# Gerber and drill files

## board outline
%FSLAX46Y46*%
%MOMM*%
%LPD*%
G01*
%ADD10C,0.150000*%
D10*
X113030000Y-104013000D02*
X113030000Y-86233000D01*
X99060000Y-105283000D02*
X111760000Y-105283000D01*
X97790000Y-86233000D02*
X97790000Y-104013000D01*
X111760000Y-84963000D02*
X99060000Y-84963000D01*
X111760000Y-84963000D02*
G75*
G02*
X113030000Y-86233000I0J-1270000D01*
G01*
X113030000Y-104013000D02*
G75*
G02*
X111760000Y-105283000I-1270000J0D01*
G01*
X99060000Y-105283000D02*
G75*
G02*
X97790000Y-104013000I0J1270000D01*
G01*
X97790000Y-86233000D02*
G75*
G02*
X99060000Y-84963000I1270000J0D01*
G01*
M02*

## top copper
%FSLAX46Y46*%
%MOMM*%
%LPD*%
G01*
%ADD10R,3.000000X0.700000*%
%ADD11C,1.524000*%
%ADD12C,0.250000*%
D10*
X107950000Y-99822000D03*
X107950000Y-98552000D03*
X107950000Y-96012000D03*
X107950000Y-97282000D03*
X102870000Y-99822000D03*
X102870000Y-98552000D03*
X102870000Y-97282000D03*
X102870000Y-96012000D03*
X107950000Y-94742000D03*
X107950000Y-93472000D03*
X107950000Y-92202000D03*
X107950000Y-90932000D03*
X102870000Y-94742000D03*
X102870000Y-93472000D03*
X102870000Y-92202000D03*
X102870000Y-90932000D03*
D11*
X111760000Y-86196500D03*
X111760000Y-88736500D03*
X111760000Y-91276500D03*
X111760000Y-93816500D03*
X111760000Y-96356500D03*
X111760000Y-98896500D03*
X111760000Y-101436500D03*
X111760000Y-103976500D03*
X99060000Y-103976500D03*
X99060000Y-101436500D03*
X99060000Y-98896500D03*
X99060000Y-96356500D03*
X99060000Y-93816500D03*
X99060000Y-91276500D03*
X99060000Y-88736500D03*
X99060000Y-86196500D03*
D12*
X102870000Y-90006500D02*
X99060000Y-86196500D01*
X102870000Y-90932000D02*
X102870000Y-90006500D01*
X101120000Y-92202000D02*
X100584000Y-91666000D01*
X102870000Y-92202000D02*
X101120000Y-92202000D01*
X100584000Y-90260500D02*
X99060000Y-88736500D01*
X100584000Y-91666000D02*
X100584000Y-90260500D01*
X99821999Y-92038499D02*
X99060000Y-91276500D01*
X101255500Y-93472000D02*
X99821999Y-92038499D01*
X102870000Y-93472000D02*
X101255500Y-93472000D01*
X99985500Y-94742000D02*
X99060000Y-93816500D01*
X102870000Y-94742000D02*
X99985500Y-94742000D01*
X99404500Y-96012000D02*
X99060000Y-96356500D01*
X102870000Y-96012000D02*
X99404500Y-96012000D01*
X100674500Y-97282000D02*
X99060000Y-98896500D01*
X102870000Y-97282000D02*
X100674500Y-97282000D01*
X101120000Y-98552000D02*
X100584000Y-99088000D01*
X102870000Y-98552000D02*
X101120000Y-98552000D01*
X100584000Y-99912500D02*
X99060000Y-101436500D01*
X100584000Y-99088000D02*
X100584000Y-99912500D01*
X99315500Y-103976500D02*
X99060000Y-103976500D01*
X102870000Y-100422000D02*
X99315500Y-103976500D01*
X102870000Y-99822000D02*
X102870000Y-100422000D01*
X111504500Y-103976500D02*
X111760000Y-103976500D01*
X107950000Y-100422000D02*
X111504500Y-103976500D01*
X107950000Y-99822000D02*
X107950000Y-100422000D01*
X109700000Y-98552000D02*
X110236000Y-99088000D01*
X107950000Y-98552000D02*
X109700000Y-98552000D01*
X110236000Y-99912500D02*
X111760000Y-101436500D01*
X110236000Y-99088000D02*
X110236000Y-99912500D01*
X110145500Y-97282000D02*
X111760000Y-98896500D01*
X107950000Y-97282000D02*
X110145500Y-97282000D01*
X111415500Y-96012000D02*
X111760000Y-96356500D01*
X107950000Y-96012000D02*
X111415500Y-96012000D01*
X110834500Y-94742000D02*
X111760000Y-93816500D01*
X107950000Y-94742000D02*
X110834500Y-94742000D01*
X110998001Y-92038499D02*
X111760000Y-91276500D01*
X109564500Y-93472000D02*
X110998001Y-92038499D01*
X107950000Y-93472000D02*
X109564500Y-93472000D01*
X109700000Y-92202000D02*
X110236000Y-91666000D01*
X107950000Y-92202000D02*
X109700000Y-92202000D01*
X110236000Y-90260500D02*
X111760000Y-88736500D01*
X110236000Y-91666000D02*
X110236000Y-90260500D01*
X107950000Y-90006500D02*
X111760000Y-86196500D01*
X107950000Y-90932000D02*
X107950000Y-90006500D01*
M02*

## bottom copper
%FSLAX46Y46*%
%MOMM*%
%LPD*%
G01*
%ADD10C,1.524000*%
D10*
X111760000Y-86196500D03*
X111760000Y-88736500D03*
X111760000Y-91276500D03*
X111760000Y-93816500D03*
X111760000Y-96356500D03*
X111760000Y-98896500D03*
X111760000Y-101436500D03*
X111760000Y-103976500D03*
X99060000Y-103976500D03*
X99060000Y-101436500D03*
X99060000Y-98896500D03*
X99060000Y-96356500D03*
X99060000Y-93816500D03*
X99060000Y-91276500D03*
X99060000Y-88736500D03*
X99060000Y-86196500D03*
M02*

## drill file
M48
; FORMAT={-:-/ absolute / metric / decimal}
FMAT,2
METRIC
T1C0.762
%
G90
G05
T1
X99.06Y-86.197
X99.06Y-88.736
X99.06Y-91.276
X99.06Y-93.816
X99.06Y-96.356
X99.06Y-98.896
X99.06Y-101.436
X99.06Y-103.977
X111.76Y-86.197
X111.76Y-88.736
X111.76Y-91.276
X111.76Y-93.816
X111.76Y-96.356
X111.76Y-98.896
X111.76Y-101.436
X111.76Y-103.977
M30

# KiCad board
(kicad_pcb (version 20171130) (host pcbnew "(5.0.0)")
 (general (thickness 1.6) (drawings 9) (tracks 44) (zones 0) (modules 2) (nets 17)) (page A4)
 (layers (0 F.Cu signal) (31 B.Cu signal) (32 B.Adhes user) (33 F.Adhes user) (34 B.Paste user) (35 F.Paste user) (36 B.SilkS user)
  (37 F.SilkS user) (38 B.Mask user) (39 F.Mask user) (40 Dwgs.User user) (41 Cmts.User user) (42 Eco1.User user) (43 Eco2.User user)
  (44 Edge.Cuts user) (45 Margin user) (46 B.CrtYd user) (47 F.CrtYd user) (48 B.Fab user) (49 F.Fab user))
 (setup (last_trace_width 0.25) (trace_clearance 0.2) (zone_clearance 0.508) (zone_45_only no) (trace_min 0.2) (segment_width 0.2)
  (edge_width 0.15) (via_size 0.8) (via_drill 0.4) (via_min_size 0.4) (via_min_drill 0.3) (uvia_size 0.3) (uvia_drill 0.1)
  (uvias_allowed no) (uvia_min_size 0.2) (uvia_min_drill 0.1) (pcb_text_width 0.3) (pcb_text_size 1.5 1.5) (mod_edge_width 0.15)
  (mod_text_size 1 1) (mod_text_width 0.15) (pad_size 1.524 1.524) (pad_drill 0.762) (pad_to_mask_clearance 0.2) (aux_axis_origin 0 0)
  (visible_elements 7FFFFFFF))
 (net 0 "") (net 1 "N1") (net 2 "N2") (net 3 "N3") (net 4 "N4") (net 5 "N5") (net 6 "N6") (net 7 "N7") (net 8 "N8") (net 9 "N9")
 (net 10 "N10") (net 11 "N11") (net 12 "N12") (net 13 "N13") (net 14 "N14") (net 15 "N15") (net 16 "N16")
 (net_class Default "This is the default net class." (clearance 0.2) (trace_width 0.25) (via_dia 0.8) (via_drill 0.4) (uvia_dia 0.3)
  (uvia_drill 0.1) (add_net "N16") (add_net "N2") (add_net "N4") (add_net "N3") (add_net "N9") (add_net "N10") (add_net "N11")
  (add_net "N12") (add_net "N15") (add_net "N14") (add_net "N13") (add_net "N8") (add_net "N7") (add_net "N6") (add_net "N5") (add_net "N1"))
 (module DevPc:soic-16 (layer F.Cu) (at 105.41 89.662)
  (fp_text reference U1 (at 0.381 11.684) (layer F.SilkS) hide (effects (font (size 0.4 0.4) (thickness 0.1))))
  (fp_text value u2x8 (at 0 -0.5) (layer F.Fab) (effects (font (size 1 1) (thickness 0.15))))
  (pad 9 smd rect (at 2.54 10.16 90) (size 0.7 3) (layers F.Cu F.Paste F.Mask) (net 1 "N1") (solder_mask_margin 0.1))
  (pad 10 smd rect (at 2.54 8.89 90) (size 0.7 3) (layers F.Cu F.Paste F.Mask) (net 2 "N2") (solder_mask_margin 0.1))
  (pad 12 smd rect (at 2.54 6.35 90) (size 0.7 3) (layers F.Cu F.Paste F.Mask) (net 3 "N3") (solder_mask_margin 0.1))
  (pad 11 smd rect (at 2.54 7.62 90) (size 0.7 3) (layers F.Cu F.Paste F.Mask) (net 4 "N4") (solder_mask_margin 0.1))
  (pad 8 smd rect (at -2.54 10.16 90) (size 0.7 3) (layers F.Cu F.Paste F.Mask) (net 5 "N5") (solder_mask_margin 0.1))
  (pad 7 smd rect (at -2.54 8.89 90) (size 0.7 3) (layers F.Cu F.Paste F.Mask) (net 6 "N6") (solder_mask_margin 0.1))
  (pad 6 smd rect (at -2.54 7.62 90) (size 0.7 3) (layers F.Cu F.Paste F.Mask) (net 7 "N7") (solder_mask_margin 0.1))
  (pad 5 smd rect (at -2.54 6.35 90) (size 0.7 3) (layers F.Cu F.Paste F.Mask) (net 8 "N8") (solder_mask_margin 0.1))
  (pad 13 smd rect (at 2.54 5.08 90) (size 0.7 3) (layers F.Cu F.Paste F.Mask) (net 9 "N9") (solder_mask_margin 0.1))
  (pad 14 smd rect (at 2.54 3.81 90) (size 0.7 3) (layers F.Cu F.Paste F.Mask) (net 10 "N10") (solder_mask_margin 0.1))
  (pad 15 smd rect (at 2.54 2.54 90) (size 0.7 3) (layers F.Cu F.Paste F.Mask) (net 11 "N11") (solder_mask_margin 0.1))
  (pad 16 smd rect (at 2.54 1.27 90) (size 0.7 3) (layers F.Cu F.Paste F.Mask) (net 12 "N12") (solder_mask_margin 0.1))
  (pad 4 smd rect (at -2.54 5.08 90) (size 0.7 3) (layers F.Cu F.Paste F.Mask) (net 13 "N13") (solder_mask_margin 0.1))
  (pad 3 smd rect (at -2.54 3.81 90) (size 0.7 3) (layers F.Cu F.Paste F.Mask) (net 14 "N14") (solder_mask_margin 0.1))
  (pad 2 smd rect (at -2.54 2.54 90) (size 0.7 3) (layers F.Cu F.Paste F.Mask) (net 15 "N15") (solder_mask_margin 0.1))
  (pad 1 smd rect (at -2.54 1.27 90) (size 0.7 3) (layers F.Cu F.Paste F.Mask) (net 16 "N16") (solder_mask_margin 0.1)))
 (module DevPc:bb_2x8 (layer F.Cu) (at 99.06 86.1965)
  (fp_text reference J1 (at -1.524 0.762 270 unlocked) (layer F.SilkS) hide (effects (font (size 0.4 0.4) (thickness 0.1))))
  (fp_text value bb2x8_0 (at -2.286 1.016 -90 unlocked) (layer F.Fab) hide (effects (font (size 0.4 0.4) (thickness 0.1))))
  (pad 16 thru_hole circle (at 12.7 0) (size 1.524 1.524) (drill 0.762) (layers *.Cu *.Mask) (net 12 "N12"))
  (pad 15 thru_hole circle (at 12.7 2.54) (size 1.524 1.524) (drill 0.762) (layers *.Cu *.Mask) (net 11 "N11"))
  (pad 14 thru_hole circle (at 12.7 5.08) (size 1.524 1.524) (drill 0.762) (layers *.Cu *.Mask) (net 10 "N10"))
  (pad 13 thru_hole circle (at 12.7 7.62) (size 1.524 1.524) (drill 0.762) (layers *.Cu *.Mask) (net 9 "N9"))
  (pad 12 thru_hole circle (at 12.7 10.16) (size 1.524 1.524) (drill 0.762) (layers *.Cu *.Mask) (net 3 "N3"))
  (pad 11 thru_hole circle (at 12.7 12.7) (size 1.524 1.524) (drill 0.762) (layers *.Cu *.Mask) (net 4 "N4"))
  (pad 10 thru_hole circle (at 12.7 15.24) (size 1.524 1.524) (drill 0.762) (layers *.Cu *.Mask) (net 2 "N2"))
  (pad 9 thru_hole circle (at 12.7 17.78) (size 1.524 1.524) (drill 0.762) (layers *.Cu *.Mask) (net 1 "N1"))
  (pad 8 thru_hole circle (at 0 17.78) (size 1.524 1.524) (drill 0.762) (layers *.Cu *.Mask) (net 5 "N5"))
  (pad 7 thru_hole circle (at 0 15.24) (size 1.524 1.524) (drill 0.762) (layers *.Cu *.Mask) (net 6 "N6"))
  (pad 6 thru_hole circle (at 0 12.7) (size 1.524 1.524) (drill 0.762) (layers *.Cu *.Mask) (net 7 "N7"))
  (pad 5 thru_hole circle (at 0 10.16) (size 1.524 1.524) (drill 0.762) (layers *.Cu *.Mask) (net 8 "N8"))
  (pad 4 thru_hole circle (at 0 7.62) (size 1.524 1.524) (drill 0.762) (layers *.Cu *.Mask) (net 13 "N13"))
  (pad 3 thru_hole circle (at 0 5.08) (size 1.524 1.524) (drill 0.762) (layers *.Cu *.Mask) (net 14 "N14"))
  (pad 2 thru_hole circle (at 0 2.54) (size 1.524 1.524) (drill 0.762) (layers *.Cu *.Mask) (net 15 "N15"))
  (pad 1 thru_hole circle (at 0 0) (size 1.524 1.524) (drill 0.762) (layers *.Cu *.Mask) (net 16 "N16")))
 (gr_line (start 113.03 104.013) (end 113.03 86.233) (layer Edge.Cuts) (width 0.15))
 (gr_line (start 99.06 105.283) (end 111.76 105.283) (layer Edge.Cuts) (width 0.15))
 (gr_line (start 97.79 86.233) (end 97.79 104.013) (layer Edge.Cuts) (width 0.15))
 (gr_line (start 111.76 84.963) (end 99.06 84.963) (layer Edge.Cuts) (width 0.15))
 (gr_arc (start 111.76 86.233) (end 113.03 86.233) (angle -90) (layer Edge.Cuts) (width 0.15))
 (gr_arc (start 111.76 104.013) (end 111.76 105.283) (angle -90) (layer Edge.Cuts) (width 0.15))
 (gr_arc (start 99.06 104.013) (end 97.79 104.013) (angle -90) (layer Edge.Cuts) (width 0.15))
 (gr_arc (start 99.06 86.233) (end 99.06 84.963) (angle -90) (layer Edge.Cuts) (width 0.15))
 (segment (start 102.87 90.0065) (end 99.06 86.1965) (width 0.25) (layer F.Cu) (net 16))
 (segment (start 102.87 90.932) (end 102.87 90.0065) (width 0.25) (layer F.Cu) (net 16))
 (segment (start 101.12 92.202) (end 100.584 91.666) (width 0.25) (layer F.Cu) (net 15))
 (segment (start 102.87 92.202) (end 101.12 92.202) (width 0.25) (layer F.Cu) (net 15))
 (segment (start 100.584 90.2605) (end 99.06 88.7365) (width 0.25) (layer F.Cu) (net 15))
 (segment (start 100.584 91.666) (end 100.584 90.2605) (width 0.25) (layer F.Cu) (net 15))
 (segment (start 99.821999 92.038499) (end 99.06 91.2765) (width 0.25) (layer F.Cu) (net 14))
 (segment (start 101.2555 93.472) (end 99.821999 92.038499) (width 0.25) (layer F.Cu) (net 14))
 (segment (start 102.87 93.472) (end 101.2555 93.472) (width 0.25) (layer F.Cu) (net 14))
 (segment (start 99.9855 94.742) (end 99.06 93.8165) (width 0.25) (layer F.Cu) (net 13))
 (segment (start 102.87 94.742) (end 99.9855 94.742) (width 0.25) (layer F.Cu) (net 13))
 (segment (start 99.4045 96.012) (end 99.06 96.3565) (width 0.25) (layer F.Cu) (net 8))
 (segment (start 102.87 96.012) (end 99.4045 96.012) (width 0.25) (layer F.Cu) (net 8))
 (segment (start 100.6745 97.282) (end 99.06 98.8965) (width 0.25) (layer F.Cu) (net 7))
 (segment (start 102.87 97.282) (end 100.6745 97.282) (width 0.25) (layer F.Cu) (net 7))
 (segment (start 101.12 98.552) (end 100.584 99.088) (width 0.25) (layer F.Cu) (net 6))
 (segment (start 102.87 98.552) (end 101.12 98.552) (width 0.25) (layer F.Cu) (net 6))
 (segment (start 100.584 99.9125) (end 99.06 101.4365) (width 0.25) (layer F.Cu) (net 6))
 (segment (start 100.584 99.088) (end 100.584 99.9125) (width 0.25) (layer F.Cu) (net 6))
 (segment (start 99.3155 103.9765) (end 99.06 103.9765) (width 0.25) (layer F.Cu) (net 5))
 (segment (start 102.87 100.422) (end 99.3155 103.9765) (width 0.25) (layer F.Cu) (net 5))
 (segment (start 102.87 99.822) (end 102.87 100.422) (width 0.25) (layer F.Cu) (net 5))
 (segment (start 111.5045 103.9765) (end 111.76 103.9765) (width 0.25) (layer F.Cu) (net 1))
 (segment (start 107.95 100.422) (end 111.5045 103.9765) (width 0.25) (layer F.Cu) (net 1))
 (segment (start 107.95 99.822) (end 107.95 100.422) (width 0.25) (layer F.Cu) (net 1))
 (segment (start 109.7 98.552) (end 110.236 99.088) (width 0.25) (layer F.Cu) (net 2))
 (segment (start 107.95 98.552) (end 109.7 98.552) (width 0.25) (layer F.Cu) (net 2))
 (segment (start 110.236 99.9125) (end 111.76 101.4365) (width 0.25) (layer F.Cu) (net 2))
 (segment (start 110.236 99.088) (end 110.236 99.9125) (width 0.25) (layer F.Cu) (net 2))
 (segment (start 110.1455 97.282) (end 111.76 98.8965) (width 0.25) (layer F.Cu) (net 4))
 (segment (start 107.95 97.282) (end 110.1455 97.282) (width 0.25) (layer F.Cu) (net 4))
 (segment (start 111.4155 96.012) (end 111.76 96.3565) (width 0.25) (layer F.Cu) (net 3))
 (segment (start 107.95 96.012) (end 111.4155 96.012) (width 0.25) (layer F.Cu) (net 3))
 (segment (start 110.8345 94.742) (end 111.76 93.8165) (width 0.25) (layer F.Cu) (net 9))
 (segment (start 107.95 94.742) (end 110.8345 94.742) (width 0.25) (layer F.Cu) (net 9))
 (segment (start 110.998001 92.038499) (end 111.76 91.2765) (width 0.25) (layer F.Cu) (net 10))
 (segment (start 109.5645 93.472) (end 110.998001 92.038499) (width 0.25) (layer F.Cu) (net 10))
 (segment (start 107.95 93.472) (end 109.5645 93.472) (width 0.25) (layer F.Cu) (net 10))
 (segment (start 109.7 92.202) (end 110.236 91.666) (width 0.25) (layer F.Cu) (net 11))
 (segment (start 107.95 92.202) (end 109.7 92.202) (width 0.25) (layer F.Cu) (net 11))
 (segment (start 110.236 90.2605) (end 111.76 88.7365) (width 0.25) (layer F.Cu) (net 11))
 (segment (start 110.236 91.666) (end 110.236 90.2605) (width 0.25) (layer F.Cu) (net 11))
 (segment (start 107.95 90.0065) (end 111.76 86.1965) (width 0.25) (layer F.Cu) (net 12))
 (segment (start 107.95 90.932) (end 107.95 90.0065) (width 0.25) (layer F.Cu) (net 12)))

